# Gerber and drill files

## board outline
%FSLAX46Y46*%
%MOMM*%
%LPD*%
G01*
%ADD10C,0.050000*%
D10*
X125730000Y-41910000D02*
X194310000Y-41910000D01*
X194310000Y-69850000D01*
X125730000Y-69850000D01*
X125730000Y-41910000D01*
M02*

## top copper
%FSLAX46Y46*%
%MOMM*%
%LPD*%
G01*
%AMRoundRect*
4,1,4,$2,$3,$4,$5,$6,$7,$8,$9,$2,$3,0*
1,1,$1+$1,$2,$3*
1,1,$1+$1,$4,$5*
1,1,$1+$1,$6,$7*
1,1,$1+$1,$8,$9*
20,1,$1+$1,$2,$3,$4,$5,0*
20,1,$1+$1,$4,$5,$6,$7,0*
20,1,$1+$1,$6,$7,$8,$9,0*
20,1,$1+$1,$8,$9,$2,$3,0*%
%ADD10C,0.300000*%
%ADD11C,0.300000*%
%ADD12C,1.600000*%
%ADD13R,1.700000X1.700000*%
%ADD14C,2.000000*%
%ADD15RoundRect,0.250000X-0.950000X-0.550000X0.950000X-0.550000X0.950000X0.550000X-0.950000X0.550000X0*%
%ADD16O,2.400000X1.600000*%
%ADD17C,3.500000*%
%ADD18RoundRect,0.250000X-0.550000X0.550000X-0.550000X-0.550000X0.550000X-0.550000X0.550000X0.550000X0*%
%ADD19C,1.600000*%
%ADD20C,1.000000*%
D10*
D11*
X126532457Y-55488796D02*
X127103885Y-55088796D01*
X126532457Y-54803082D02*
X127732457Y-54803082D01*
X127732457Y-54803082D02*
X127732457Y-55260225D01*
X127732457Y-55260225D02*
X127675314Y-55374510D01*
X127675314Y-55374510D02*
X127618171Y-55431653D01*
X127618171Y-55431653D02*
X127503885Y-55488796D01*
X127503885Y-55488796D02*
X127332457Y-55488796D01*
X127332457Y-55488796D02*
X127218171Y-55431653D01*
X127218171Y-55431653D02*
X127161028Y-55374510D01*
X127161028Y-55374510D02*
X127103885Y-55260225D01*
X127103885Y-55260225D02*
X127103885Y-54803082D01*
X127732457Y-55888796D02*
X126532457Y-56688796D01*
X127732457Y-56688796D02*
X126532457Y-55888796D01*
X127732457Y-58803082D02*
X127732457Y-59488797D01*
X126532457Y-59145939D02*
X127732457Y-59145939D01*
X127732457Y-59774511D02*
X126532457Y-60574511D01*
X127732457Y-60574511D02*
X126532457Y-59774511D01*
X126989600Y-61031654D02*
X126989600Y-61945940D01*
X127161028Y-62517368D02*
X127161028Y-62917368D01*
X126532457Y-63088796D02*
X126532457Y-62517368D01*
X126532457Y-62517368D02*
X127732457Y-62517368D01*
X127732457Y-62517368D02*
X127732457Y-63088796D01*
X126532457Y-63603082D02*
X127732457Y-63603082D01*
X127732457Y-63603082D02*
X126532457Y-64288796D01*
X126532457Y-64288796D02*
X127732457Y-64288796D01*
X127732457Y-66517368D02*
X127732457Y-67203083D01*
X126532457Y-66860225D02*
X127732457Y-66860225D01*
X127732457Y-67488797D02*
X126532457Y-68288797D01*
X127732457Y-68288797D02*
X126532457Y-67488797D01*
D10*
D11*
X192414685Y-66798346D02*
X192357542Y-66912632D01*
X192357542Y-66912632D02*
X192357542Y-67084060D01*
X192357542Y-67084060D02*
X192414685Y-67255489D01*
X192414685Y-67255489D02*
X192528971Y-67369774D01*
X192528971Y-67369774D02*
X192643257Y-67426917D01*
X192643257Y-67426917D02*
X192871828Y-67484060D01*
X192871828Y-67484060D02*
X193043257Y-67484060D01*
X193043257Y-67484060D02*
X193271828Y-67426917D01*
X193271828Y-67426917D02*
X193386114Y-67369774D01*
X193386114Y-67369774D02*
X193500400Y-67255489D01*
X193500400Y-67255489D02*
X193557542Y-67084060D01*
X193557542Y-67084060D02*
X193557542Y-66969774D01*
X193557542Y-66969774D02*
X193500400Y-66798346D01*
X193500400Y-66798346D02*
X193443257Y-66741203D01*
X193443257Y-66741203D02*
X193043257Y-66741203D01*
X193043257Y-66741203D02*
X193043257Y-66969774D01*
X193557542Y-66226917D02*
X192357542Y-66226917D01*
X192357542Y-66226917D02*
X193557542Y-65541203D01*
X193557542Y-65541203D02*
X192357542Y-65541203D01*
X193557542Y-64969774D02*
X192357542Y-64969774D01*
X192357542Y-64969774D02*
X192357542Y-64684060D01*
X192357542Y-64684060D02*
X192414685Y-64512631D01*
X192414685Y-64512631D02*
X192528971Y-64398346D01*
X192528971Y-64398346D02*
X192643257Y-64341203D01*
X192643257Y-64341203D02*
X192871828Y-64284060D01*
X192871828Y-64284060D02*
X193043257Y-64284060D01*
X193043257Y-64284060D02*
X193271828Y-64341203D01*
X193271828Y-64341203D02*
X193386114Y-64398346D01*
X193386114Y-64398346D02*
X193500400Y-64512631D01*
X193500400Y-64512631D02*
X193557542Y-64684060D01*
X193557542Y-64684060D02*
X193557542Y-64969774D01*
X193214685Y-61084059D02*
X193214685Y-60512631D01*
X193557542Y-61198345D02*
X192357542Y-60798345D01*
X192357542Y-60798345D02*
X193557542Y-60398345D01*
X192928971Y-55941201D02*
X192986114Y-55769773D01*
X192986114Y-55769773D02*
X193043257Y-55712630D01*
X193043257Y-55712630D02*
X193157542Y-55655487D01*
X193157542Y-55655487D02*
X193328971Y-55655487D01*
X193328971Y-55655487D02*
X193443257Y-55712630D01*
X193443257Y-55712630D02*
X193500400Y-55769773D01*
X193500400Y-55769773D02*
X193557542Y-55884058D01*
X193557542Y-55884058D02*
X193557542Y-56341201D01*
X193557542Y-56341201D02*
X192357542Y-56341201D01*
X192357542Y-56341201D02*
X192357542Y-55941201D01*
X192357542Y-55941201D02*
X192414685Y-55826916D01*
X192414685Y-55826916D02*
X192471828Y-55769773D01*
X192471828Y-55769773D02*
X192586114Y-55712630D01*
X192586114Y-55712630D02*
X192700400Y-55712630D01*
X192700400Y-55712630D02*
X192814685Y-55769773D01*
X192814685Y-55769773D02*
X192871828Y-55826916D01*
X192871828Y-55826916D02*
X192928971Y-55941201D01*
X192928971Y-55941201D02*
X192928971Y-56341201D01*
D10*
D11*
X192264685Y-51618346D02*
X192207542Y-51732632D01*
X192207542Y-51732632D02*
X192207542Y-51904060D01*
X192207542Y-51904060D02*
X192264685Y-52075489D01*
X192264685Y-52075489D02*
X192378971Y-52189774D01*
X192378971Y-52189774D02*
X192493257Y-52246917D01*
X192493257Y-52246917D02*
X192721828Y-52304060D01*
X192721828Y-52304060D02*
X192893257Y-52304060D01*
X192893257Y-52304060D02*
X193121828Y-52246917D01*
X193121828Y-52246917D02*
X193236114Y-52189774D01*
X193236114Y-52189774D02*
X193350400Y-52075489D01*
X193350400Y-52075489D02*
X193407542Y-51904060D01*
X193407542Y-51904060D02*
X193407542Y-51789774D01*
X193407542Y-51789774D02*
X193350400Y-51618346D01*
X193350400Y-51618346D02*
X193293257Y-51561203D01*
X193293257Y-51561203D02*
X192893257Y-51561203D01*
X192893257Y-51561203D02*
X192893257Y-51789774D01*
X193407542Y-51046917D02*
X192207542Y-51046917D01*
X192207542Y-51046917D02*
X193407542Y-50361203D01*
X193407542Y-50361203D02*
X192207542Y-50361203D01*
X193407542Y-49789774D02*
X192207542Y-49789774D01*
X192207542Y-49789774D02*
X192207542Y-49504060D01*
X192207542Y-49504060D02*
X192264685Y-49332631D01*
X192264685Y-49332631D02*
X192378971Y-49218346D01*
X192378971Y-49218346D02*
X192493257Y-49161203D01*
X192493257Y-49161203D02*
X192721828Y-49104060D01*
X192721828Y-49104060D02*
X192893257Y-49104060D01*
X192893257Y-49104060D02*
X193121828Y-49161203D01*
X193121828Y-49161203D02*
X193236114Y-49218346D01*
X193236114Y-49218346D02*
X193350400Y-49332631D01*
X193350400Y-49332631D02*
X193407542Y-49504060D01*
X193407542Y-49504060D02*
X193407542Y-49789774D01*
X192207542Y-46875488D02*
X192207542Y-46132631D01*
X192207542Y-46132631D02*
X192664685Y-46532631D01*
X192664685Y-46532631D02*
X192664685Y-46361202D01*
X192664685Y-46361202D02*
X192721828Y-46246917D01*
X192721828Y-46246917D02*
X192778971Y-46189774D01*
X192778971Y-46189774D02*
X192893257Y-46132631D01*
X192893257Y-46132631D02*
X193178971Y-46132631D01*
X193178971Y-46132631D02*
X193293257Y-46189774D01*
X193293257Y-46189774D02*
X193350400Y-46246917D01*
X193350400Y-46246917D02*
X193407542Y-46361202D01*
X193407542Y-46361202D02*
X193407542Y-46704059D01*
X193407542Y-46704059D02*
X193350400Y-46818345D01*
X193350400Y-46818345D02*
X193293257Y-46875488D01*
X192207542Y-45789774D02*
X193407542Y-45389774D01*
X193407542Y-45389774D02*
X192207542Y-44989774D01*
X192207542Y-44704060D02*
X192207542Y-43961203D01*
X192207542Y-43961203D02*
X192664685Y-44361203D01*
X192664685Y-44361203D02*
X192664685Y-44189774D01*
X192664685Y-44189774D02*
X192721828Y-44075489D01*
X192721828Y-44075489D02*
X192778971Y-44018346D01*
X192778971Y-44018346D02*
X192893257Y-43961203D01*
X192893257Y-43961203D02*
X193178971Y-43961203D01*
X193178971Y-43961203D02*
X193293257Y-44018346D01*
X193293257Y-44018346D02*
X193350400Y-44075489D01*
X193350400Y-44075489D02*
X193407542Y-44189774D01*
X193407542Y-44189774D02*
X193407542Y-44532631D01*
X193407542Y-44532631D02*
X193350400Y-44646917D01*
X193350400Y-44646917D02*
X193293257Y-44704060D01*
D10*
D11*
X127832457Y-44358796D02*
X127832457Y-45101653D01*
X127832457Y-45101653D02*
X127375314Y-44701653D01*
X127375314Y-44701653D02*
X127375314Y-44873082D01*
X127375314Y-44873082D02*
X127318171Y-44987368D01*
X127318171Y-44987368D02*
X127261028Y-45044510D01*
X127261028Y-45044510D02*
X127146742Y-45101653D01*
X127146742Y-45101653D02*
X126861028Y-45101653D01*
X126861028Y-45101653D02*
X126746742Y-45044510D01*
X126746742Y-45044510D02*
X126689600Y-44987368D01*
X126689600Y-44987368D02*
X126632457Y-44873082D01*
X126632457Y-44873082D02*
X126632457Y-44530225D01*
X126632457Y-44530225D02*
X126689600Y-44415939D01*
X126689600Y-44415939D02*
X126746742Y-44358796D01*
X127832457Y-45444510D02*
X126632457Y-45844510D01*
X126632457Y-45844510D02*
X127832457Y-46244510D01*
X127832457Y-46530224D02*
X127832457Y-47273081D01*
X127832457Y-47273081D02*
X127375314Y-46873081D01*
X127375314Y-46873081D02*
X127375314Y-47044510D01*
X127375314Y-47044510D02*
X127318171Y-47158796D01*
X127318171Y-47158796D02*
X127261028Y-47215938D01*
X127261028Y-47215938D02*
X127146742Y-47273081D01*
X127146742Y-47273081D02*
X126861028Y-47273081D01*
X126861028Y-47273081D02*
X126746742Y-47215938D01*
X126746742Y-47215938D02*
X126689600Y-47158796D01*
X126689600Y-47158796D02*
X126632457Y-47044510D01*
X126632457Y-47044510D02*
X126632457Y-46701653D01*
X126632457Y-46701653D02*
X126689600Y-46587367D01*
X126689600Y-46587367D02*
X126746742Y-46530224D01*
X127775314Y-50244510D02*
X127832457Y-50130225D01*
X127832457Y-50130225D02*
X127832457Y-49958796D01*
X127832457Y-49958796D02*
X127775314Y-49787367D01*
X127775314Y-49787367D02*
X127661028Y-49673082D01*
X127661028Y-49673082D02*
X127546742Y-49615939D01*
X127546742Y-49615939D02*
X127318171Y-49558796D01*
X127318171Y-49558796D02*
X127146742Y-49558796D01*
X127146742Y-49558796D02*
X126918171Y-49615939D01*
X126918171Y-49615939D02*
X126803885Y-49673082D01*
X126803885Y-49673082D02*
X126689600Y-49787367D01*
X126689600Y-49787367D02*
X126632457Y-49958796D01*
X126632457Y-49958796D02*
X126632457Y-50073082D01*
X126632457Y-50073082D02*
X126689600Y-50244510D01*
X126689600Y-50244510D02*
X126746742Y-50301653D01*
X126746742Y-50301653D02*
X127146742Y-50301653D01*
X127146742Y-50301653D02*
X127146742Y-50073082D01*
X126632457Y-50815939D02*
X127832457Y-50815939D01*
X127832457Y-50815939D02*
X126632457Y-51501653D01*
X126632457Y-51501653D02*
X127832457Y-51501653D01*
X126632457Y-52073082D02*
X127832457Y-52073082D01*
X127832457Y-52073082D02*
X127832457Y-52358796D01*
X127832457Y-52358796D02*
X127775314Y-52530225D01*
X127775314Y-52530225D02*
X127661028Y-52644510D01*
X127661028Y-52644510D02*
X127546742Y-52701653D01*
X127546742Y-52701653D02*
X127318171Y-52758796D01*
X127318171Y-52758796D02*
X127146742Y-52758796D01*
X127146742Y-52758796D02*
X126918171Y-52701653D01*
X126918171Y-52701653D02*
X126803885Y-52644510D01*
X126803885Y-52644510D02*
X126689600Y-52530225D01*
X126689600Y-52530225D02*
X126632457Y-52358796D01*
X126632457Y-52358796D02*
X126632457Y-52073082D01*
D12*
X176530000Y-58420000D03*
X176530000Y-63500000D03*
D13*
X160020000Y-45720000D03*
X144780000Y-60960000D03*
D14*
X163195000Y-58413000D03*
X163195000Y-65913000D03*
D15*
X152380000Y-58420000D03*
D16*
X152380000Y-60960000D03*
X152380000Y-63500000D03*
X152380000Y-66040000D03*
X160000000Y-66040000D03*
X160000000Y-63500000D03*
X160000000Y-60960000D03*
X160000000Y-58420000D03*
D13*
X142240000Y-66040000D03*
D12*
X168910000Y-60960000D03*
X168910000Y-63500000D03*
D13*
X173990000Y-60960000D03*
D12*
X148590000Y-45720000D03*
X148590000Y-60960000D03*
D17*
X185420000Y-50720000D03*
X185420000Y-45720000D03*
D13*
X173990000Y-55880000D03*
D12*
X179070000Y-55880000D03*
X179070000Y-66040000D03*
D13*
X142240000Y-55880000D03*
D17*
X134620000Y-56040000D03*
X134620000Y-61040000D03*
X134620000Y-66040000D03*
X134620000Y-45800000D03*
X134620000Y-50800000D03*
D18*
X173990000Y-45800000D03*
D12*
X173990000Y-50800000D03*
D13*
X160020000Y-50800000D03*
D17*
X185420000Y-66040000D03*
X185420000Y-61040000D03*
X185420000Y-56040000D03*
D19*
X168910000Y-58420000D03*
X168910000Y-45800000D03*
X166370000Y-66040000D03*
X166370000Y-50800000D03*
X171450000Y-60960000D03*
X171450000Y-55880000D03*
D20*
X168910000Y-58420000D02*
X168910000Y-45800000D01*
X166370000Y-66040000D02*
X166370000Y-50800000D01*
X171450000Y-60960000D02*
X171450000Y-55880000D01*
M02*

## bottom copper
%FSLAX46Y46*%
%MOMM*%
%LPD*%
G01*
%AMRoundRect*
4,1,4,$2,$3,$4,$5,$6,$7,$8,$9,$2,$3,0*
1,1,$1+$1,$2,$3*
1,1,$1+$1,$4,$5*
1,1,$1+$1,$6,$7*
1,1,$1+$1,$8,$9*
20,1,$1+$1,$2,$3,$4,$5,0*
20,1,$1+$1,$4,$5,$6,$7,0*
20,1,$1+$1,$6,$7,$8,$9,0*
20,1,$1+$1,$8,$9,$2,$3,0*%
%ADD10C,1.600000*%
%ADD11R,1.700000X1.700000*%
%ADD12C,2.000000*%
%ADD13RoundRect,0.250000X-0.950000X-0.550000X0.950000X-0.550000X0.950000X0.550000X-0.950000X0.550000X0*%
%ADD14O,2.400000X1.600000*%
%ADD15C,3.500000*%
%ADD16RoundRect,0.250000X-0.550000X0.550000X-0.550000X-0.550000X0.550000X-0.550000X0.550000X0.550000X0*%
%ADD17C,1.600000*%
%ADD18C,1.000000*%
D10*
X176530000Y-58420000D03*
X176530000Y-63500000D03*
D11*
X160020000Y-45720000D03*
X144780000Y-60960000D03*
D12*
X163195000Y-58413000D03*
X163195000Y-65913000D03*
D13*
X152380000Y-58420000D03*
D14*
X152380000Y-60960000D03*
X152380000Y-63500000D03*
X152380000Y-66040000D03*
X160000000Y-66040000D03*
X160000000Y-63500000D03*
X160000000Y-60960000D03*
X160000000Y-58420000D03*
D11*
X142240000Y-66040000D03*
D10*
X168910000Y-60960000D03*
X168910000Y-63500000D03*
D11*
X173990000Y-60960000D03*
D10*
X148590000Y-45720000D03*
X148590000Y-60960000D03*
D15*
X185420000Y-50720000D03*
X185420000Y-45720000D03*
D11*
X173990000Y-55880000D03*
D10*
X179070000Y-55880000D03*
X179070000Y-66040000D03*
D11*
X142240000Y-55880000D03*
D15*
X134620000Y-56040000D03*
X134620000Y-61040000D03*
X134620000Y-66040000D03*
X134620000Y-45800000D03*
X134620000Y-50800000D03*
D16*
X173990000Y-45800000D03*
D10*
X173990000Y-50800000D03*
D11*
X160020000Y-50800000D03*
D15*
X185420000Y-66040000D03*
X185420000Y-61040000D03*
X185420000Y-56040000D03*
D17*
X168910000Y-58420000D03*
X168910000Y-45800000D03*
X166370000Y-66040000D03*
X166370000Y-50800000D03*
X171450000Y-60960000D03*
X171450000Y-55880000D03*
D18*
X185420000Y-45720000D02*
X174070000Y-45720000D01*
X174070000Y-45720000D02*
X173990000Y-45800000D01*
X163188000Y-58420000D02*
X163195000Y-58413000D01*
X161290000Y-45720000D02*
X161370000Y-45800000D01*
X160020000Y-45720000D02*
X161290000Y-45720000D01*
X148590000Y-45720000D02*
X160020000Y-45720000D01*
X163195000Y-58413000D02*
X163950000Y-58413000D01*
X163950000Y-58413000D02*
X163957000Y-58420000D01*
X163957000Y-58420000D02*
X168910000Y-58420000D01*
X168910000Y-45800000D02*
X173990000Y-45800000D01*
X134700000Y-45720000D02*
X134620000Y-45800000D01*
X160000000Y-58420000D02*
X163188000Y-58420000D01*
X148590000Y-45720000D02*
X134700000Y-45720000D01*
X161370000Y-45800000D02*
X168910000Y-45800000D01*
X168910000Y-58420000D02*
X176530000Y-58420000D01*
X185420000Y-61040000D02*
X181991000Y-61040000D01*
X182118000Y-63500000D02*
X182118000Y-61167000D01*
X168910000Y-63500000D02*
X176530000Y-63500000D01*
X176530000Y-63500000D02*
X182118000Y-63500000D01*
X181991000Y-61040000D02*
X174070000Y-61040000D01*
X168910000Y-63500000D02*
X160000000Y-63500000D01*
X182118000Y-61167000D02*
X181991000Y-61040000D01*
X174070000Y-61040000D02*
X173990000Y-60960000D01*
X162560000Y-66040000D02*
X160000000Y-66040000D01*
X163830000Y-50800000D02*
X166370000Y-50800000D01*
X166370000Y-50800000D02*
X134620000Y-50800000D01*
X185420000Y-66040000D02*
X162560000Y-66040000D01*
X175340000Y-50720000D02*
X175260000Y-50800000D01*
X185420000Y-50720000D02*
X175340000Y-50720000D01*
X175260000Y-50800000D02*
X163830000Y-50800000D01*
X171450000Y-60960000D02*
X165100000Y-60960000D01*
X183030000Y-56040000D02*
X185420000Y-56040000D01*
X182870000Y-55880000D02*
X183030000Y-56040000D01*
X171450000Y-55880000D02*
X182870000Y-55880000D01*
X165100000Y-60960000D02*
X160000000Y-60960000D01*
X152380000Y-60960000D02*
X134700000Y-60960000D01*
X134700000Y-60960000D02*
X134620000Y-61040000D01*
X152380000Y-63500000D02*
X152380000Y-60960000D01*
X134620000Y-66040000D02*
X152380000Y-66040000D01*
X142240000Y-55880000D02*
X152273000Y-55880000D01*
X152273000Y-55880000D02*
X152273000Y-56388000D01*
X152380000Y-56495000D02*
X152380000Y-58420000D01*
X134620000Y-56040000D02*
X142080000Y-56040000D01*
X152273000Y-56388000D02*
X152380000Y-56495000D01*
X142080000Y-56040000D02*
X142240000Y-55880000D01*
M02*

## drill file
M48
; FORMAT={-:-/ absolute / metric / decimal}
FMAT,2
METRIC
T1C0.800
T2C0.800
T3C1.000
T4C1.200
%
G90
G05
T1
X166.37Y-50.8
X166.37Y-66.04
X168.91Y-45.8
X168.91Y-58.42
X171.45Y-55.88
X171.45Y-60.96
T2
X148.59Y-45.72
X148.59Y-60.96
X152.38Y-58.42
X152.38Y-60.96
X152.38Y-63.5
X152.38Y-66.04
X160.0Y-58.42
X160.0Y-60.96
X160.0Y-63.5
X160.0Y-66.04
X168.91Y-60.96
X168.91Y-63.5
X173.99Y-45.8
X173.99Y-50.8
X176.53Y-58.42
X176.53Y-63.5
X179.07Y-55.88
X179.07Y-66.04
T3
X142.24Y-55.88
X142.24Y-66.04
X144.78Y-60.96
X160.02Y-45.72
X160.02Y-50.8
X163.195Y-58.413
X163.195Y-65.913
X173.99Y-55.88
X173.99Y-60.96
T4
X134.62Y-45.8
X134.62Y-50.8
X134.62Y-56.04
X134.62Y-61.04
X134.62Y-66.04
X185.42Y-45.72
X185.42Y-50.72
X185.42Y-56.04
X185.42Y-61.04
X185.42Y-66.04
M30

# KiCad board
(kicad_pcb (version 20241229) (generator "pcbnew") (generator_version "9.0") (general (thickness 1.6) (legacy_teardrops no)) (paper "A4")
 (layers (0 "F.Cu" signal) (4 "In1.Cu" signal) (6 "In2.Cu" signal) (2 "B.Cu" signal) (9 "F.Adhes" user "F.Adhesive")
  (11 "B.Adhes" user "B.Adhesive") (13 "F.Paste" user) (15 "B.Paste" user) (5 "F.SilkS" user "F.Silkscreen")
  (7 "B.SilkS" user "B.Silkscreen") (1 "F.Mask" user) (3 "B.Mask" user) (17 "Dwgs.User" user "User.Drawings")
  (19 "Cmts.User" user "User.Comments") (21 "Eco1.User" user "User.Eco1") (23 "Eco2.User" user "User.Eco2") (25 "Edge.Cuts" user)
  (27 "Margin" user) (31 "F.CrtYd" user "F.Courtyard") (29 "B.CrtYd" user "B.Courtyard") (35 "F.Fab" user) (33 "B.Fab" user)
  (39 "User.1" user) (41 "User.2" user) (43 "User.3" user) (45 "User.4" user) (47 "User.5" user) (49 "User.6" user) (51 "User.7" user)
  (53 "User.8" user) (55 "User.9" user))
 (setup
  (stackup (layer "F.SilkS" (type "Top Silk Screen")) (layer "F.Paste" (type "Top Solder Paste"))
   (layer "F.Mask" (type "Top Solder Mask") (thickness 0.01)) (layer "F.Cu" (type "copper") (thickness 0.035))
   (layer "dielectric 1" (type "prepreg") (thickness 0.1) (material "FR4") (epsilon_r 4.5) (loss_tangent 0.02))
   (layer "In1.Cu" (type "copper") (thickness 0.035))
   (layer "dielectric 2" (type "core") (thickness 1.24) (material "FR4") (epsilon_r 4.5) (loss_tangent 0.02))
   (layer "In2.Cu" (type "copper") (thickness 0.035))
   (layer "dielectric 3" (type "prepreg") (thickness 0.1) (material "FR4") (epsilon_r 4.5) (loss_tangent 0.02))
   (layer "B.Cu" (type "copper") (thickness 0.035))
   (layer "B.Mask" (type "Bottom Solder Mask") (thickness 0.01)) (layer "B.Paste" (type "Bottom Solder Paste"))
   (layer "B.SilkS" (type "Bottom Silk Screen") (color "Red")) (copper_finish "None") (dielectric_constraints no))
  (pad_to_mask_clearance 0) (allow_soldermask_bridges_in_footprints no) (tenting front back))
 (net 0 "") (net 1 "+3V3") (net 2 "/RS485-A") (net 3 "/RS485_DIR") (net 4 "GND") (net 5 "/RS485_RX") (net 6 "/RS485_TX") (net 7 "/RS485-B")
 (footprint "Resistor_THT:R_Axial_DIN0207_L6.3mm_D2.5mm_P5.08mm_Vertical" (layer "F.Cu") (at 176.53 58.42 -90)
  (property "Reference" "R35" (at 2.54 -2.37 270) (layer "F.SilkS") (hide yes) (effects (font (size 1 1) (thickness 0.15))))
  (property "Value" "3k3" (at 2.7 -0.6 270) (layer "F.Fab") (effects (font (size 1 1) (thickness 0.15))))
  (pad "1" thru_hole circle (at 0 0 270) (size 1.6 1.6) (drill 0.8) (layers "*.Cu" "*.Mask") (remove_unused_layers no) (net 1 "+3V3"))
  (pad "2" thru_hole circle (at 5.08 0 270) (size 1.6 1.6) (drill 0.8) (layers "*.Cu" "*.Mask") (remove_unused_layers no) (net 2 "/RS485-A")))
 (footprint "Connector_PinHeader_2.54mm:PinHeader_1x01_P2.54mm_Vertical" (layer "F.Cu") (at 160.02 45.72)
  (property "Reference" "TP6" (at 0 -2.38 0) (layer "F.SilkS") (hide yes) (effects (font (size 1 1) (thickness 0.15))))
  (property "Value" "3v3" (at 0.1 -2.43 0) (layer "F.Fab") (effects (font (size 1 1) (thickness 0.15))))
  (pad "1" thru_hole rect (at 0 0) (size 1.7 1.7) (drill 1) (layers "*.Cu" "*.Mask") (remove_unused_layers no) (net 1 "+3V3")))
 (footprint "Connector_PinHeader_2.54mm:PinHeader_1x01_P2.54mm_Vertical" (layer "F.Cu") (at 144.78 60.96)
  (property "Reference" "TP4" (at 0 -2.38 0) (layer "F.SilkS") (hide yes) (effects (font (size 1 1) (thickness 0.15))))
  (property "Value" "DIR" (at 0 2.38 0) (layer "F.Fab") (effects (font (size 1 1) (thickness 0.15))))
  (pad "1" thru_hole rect (at 0 0) (size 1.7 1.7) (drill 1) (layers "*.Cu" "*.Mask") (remove_unused_layers no) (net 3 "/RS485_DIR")))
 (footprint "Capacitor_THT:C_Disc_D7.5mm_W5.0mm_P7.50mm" (layer "F.Cu") (at 163.195 58.413 -90)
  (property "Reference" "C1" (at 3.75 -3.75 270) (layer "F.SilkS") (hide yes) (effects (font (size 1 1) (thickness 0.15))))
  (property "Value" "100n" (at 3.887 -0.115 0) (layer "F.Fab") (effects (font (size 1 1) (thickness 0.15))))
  (pad "1" thru_hole circle (at 0 0 270) (size 2 2) (drill 1) (layers "*.Cu" "*.Mask") (remove_unused_layers no) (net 1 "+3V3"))
  (pad "2" thru_hole circle (at 7.5 0 270) (size 2 2) (drill 1) (layers "*.Cu" "*.Mask") (remove_unused_layers no) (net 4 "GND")))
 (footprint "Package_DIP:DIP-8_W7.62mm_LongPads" (layer "F.Cu") (at 152.38 58.42)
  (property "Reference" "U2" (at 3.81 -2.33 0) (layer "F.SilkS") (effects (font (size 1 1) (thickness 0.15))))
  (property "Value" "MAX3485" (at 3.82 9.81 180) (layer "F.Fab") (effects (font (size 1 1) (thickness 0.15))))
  (pad "1" thru_hole roundrect (at 0 0) (size 2.4 1.6) (drill 0.8) (layers "*.Cu" "*.Mask") (remove_unused_layers no)
   (roundrect_rratio 0.15625) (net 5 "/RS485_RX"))
  (pad "2" thru_hole oval (at 0 2.54) (size 2.4 1.6) (drill 0.8) (layers "*.Cu" "*.Mask") (remove_unused_layers no) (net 3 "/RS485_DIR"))
  (pad "3" thru_hole oval (at 0 5.08) (size 2.4 1.6) (drill 0.8) (layers "*.Cu" "*.Mask") (remove_unused_layers no) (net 3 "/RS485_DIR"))
  (pad "4" thru_hole oval (at 0 7.62) (size 2.4 1.6) (drill 0.8) (layers "*.Cu" "*.Mask") (remove_unused_layers no) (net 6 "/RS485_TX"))
  (pad "5" thru_hole oval (at 7.62 7.62) (size 2.4 1.6) (drill 0.8) (layers "*.Cu" "*.Mask") (remove_unused_layers no) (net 4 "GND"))
  (pad "6" thru_hole oval (at 7.62 5.08) (size 2.4 1.6) (drill 0.8) (layers "*.Cu" "*.Mask") (remove_unused_layers no) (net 2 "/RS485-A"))
  (pad "7" thru_hole oval (at 7.62 2.54) (size 2.4 1.6) (drill 0.8) (layers "*.Cu" "*.Mask") (remove_unused_layers no) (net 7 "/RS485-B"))
  (pad "8" thru_hole oval (at 7.62 0) (size 2.4 1.6) (drill 0.8) (layers "*.Cu" "*.Mask") (remove_unused_layers no) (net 1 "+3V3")))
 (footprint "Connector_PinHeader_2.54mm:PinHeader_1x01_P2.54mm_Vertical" (layer "F.Cu") (at 142.24 66.04)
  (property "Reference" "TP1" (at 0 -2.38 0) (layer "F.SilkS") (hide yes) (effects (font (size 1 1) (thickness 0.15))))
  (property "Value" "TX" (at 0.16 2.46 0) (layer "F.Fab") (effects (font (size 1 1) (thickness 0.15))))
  (pad "1" thru_hole rect (at 0 0) (size 1.7 1.7) (drill 1) (layers "*.Cu" "*.Mask") (remove_unused_layers no) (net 6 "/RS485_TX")))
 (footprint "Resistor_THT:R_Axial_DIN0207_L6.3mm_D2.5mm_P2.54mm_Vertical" (layer "F.Cu") (at 168.91 60.96 -90)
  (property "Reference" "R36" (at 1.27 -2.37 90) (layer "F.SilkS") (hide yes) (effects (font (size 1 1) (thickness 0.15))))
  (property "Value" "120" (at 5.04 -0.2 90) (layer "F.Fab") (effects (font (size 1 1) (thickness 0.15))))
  (pad "1" thru_hole circle (at 0 0 270) (size 1.6 1.6) (drill 0.8) (layers "*.Cu" "*.Mask") (remove_unused_layers no) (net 7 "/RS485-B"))
  (pad "2" thru_hole circle (at 2.54 0 270) (size 1.6 1.6) (drill 0.8) (layers "*.Cu" "*.Mask") (remove_unused_layers no) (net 2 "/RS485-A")))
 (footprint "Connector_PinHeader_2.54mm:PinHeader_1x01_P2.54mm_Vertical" (layer "F.Cu") (at 173.99 60.96)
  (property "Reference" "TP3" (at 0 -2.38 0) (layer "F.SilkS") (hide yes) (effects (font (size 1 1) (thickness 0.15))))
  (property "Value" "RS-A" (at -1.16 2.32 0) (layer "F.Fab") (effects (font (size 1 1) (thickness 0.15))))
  (pad "1" thru_hole rect (at 0 0) (size 1.7 1.7) (drill 1) (layers "*.Cu" "*.Mask") (remove_unused_layers no) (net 2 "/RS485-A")))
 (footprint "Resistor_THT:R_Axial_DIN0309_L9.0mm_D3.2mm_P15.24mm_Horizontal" (layer "F.Cu") (at 148.59 45.72 -90)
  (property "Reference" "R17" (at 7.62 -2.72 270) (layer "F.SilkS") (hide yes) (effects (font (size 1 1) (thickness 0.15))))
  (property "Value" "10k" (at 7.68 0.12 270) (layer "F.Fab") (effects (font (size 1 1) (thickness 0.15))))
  (pad "1" thru_hole circle (at 0 0 270) (size 1.6 1.6) (drill 0.8) (layers "*.Cu" "*.Mask") (remove_unused_layers no) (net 1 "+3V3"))
  (pad "2" thru_hole circle (at 15.24 0 270) (size 1.6 1.6) (drill 0.8) (layers "*.Cu" "*.Mask") (remove_unused_layers no)
   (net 3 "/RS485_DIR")))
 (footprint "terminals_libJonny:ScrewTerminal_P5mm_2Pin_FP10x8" (layer "F.Cu") (at 185.42 50.72 90)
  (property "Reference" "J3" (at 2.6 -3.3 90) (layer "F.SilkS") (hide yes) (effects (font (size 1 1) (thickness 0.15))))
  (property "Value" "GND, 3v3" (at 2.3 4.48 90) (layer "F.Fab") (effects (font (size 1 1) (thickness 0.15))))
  (pad "1" thru_hole circle (at 0 0 90) (size 3.5 3.5) (drill 1.2) (layers "*.Cu" "*.Mask") (remove_unused_layers no) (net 4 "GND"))
  (pad "2" thru_hole circle (at 5 0 90) (size 3.5 3.5) (drill 1.2) (layers "*.Cu" "*.Mask") (remove_unused_layers no) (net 1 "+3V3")))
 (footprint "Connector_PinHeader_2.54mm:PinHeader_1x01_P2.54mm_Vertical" (layer "F.Cu") (at 173.99 55.88)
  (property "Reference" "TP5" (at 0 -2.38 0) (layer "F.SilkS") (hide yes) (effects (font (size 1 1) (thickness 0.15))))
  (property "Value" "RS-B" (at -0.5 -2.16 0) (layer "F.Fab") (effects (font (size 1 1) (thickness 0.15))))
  (pad "1" thru_hole rect (at 0 0) (size 1.7 1.7) (drill 1) (layers "*.Cu" "*.Mask") (remove_unused_layers no) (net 7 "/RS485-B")))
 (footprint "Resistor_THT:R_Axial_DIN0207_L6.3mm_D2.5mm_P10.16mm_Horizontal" (layer "F.Cu") (at 179.07 55.88 -90)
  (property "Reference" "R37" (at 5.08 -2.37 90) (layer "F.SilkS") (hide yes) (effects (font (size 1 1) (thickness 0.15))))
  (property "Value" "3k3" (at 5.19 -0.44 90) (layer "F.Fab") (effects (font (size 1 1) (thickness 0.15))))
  (pad "1" thru_hole circle (at 0 0 270) (size 1.6 1.6) (drill 0.8) (layers "*.Cu" "*.Mask") (remove_unused_layers no) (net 7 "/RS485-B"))
  (pad "2" thru_hole circle (at 10.16 0 270) (size 1.6 1.6) (drill 0.8) (layers "*.Cu" "*.Mask") (remove_unused_layers no) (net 4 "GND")))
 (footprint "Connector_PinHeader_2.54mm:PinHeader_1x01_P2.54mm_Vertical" (layer "F.Cu") (at 142.24 55.88)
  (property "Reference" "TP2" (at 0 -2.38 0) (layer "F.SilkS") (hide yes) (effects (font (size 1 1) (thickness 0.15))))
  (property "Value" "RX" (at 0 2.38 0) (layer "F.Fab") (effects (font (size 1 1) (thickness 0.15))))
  (pad "1" thru_hole rect (at 0 0) (size 1.7 1.7) (drill 1) (layers "*.Cu" "*.Mask") (remove_unused_layers no) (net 5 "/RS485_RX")))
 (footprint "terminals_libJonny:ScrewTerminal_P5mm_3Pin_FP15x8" (layer "F.Cu") (at 134.62 56.04 -90)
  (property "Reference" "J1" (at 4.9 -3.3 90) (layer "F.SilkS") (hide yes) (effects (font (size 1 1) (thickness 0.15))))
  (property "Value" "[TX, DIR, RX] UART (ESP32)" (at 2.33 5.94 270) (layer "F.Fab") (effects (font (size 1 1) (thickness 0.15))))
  (pad "1" thru_hole circle (at 0 0 270) (size 3.5 3.5) (drill 1.2) (layers "*.Cu" "*.Mask") (remove_unused_layers no) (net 5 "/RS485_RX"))
  (pad "2" thru_hole circle (at 5 0 270) (size 3.5 3.5) (drill 1.2) (layers "*.Cu" "*.Mask") (remove_unused_layers no) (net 3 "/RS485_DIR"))
  (pad "3" thru_hole circle (at 10 0 270) (size 3.5 3.5) (drill 1.2) (layers "*.Cu" "*.Mask") (remove_unused_layers no) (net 6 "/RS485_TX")))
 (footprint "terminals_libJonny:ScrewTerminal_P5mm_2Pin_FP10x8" (layer "F.Cu") (at 134.62 45.8 -90)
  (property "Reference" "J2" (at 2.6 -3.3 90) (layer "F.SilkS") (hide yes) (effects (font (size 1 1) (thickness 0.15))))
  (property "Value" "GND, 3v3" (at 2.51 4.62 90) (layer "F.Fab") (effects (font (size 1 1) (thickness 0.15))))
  (pad "1" thru_hole circle (at 0 0 270) (size 3.5 3.5) (drill 1.2) (layers "*.Cu" "*.Mask") (remove_unused_layers no) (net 1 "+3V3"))
  (pad "2" thru_hole circle (at 5 0 270) (size 3.5 3.5) (drill 1.2) (layers "*.Cu" "*.Mask") (remove_unused_layers no) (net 4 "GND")))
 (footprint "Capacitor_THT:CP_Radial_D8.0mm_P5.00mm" (layer "F.Cu") (at 173.99 45.8 -90)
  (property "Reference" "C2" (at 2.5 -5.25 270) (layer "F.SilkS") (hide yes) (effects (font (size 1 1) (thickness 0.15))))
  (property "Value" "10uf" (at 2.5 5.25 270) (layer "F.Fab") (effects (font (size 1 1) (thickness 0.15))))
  (pad "1" thru_hole roundrect (at 0 0 270) (size 1.6 1.6) (drill 0.8) (layers "*.Cu" "*.Mask") (remove_unused_layers no)
   (roundrect_rratio 0.15625) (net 1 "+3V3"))
  (pad "2" thru_hole circle (at 5 0 270) (size 1.6 1.6) (drill 0.8) (layers "*.Cu" "*.Mask") (remove_unused_layers no) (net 4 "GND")))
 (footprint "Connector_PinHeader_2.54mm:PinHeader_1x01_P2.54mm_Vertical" (layer "F.Cu") (at 160.02 50.8)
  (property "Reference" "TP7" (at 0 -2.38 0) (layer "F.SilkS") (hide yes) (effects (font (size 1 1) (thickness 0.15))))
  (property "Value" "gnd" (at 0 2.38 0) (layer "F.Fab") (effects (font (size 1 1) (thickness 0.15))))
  (pad "1" thru_hole rect (at 0 0) (size 1.7 1.7) (drill 1) (layers "*.Cu" "*.Mask") (remove_unused_layers no) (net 4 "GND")))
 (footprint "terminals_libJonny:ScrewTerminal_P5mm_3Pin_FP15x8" (layer "F.Cu") (at 185.42 66.04 90)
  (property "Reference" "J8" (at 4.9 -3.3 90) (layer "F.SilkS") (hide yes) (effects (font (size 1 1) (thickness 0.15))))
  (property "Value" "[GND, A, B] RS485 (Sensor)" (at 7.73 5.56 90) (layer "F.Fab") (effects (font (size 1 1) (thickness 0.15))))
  (pad "1" thru_hole circle (at 0 0 90) (size 3.5 3.5) (drill 1.2) (layers "*.Cu" "*.Mask") (remove_unused_layers no) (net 4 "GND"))
  (pad "2" thru_hole circle (at 5 0 90) (size 3.5 3.5) (drill 1.2) (layers "*.Cu" "*.Mask") (remove_unused_layers no) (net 2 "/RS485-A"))
  (pad "3" thru_hole circle (at 10 0 90) (size 3.5 3.5) (drill 1.2) (layers "*.Cu" "*.Mask") (remove_unused_layers no) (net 7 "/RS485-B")))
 (gr_rect (start 125.73 41.91) (end 194.31 69.85) (stroke (width 0.05) (type default)) (fill no) (layer "Edge.Cuts"))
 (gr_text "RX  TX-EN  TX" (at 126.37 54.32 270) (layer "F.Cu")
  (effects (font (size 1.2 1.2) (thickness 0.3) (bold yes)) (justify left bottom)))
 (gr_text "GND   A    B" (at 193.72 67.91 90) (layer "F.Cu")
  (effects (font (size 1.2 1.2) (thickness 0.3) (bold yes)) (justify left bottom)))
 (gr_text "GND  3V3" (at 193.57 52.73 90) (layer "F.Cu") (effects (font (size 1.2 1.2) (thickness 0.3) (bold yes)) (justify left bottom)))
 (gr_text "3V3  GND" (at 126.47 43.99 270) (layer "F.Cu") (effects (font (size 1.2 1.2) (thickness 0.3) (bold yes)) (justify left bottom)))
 (segment (start 168.91 58.42) (end 168.91 45.8) (width 1) (layer "F.Cu") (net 1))
 (via (at 168.91 58.42) (size 1.6) (drill 0.8) (layers "F.Cu" "B.Cu") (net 1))
 (via (at 168.91 45.8) (size 1.6) (drill 0.8) (layers "F.Cu" "B.Cu") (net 1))
 (segment (start 185.42 45.72) (end 174.07 45.72) (width 1) (layer "B.Cu") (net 1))
 (segment (start 174.07 45.72) (end 173.99 45.8) (width 1) (layer "B.Cu") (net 1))
 (segment (start 163.188 58.42) (end 163.195 58.413) (width 1) (layer "B.Cu") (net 1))
 (segment (start 161.29 45.72) (end 161.37 45.8) (width 1) (layer "B.Cu") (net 1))
 (segment (start 160.02 45.72) (end 161.29 45.72) (width 1) (layer "B.Cu") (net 1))
 (segment (start 148.59 45.72) (end 160.02 45.72) (width 1) (layer "B.Cu") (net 1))
 (segment (start 163.195 58.413) (end 163.95 58.413) (width 1) (layer "B.Cu") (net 1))
 (segment (start 163.95 58.413) (end 163.957 58.42) (width 1) (layer "B.Cu") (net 1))
 (segment (start 163.957 58.42) (end 168.91 58.42) (width 1) (layer "B.Cu") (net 1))
 (segment (start 168.91 45.8) (end 173.99 45.8) (width 1) (layer "B.Cu") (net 1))
 (segment (start 134.7 45.72) (end 134.62 45.8) (width 1) (layer "B.Cu") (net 1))
 (segment (start 160 58.42) (end 163.188 58.42) (width 1) (layer "B.Cu") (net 1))
 (segment (start 148.59 45.72) (end 134.7 45.72) (width 1) (layer "B.Cu") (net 1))
 (segment (start 161.37 45.8) (end 168.91 45.8) (width 1) (layer "B.Cu") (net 1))
 (segment (start 168.91 58.42) (end 176.53 58.42) (width 1) (layer "B.Cu") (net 1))
 (segment (start 185.42 61.04) (end 181.991 61.04) (width 1) (layer "B.Cu") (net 2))
 (segment (start 182.118 63.5) (end 182.118 61.167) (width 1) (layer "B.Cu") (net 2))
 (segment (start 168.91 63.5) (end 176.53 63.5) (width 1) (layer "B.Cu") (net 2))
 (segment (start 176.53 63.5) (end 182.118 63.5) (width 1) (layer "B.Cu") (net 2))
 (segment (start 181.991 61.04) (end 174.07 61.04) (width 1) (layer "B.Cu") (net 2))
 (segment (start 168.91 63.5) (end 160 63.5) (width 1) (layer "B.Cu") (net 2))
 (segment (start 182.118 61.167) (end 181.991 61.04) (width 1) (layer "B.Cu") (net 2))
 (segment (start 174.07 61.04) (end 173.99 60.96) (width 1) (layer "B.Cu") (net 2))
 (segment (start 166.37 66.04) (end 166.37 50.8) (width 1) (layer "F.Cu") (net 4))
 (via (at 166.37 66.04) (size 1.6) (drill 0.8) (layers "F.Cu" "B.Cu") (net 4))
 (via (at 166.37 50.8) (size 1.6) (drill 0.8) (layers "F.Cu" "B.Cu") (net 4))
 (segment (start 162.56 66.04) (end 160 66.04) (width 1) (layer "B.Cu") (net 4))
 (segment (start 163.83 50.8) (end 166.37 50.8) (width 1) (layer "B.Cu") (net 4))
 (segment (start 166.37 50.8) (end 134.62 50.8) (width 1) (layer "B.Cu") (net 4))
 (segment (start 185.42 66.04) (end 162.56 66.04) (width 1) (layer "B.Cu") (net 4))
 (segment (start 175.34 50.72) (end 175.26 50.8) (width 1) (layer "B.Cu") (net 4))
 (segment (start 185.42 50.72) (end 175.34 50.72) (width 1) (layer "B.Cu") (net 4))
 (segment (start 175.26 50.8) (end 163.83 50.8) (width 1) (layer "B.Cu") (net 4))
 (segment (start 171.45 60.96) (end 171.45 55.88) (width 1) (layer "F.Cu") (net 7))
 (via (at 171.45 60.96) (size 1.6) (drill 0.8) (layers "F.Cu" "B.Cu") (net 7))
 (via (at 171.45 55.88) (size 1.6) (drill 0.8) (layers "F.Cu" "B.Cu") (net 7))
 (segment (start 171.45 60.96) (end 165.1 60.96) (width 1) (layer "B.Cu") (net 7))
 (segment (start 183.03 56.04) (end 185.42 56.04) (width 1) (layer "B.Cu") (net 7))
 (segment (start 182.87 55.88) (end 183.03 56.04) (width 1) (layer "B.Cu") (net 7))
 (segment (start 171.45 55.88) (end 182.87 55.88) (width 1) (layer "B.Cu") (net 7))
 (segment (start 165.1 60.96) (end 160 60.96) (width 1) (layer "B.Cu") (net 7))
 (segment (start 152.38 60.96) (end 134.7 60.96) (width 1) (layer "B.Cu") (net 3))
 (segment (start 134.7 60.96) (end 134.62 61.04) (width 1) (layer "B.Cu") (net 3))
 (segment (start 152.38 63.5) (end 152.38 60.96) (width 1) (layer "B.Cu") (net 3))
 (segment (start 134.62 66.04) (end 152.38 66.04) (width 1) (layer "B.Cu") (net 6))
 (segment (start 142.24 55.88) (end 152.273 55.88) (width 1) (layer "B.Cu") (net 5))
 (segment (start 152.273 55.88) (end 152.273 56.388) (width 1) (layer "B.Cu") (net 5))
 (segment (start 152.38 56.495) (end 152.38 58.42) (width 1) (layer "B.Cu") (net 5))
 (segment (start 134.62 56.04) (end 142.08 56.04) (width 1) (layer "B.Cu") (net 5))
 (segment (start 152.273 56.388) (end 152.38 56.495) (width 1) (layer "B.Cu") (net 5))
 (segment (start 142.08 56.04) (end 142.24 55.88) (width 1) (layer "B.Cu") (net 5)))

